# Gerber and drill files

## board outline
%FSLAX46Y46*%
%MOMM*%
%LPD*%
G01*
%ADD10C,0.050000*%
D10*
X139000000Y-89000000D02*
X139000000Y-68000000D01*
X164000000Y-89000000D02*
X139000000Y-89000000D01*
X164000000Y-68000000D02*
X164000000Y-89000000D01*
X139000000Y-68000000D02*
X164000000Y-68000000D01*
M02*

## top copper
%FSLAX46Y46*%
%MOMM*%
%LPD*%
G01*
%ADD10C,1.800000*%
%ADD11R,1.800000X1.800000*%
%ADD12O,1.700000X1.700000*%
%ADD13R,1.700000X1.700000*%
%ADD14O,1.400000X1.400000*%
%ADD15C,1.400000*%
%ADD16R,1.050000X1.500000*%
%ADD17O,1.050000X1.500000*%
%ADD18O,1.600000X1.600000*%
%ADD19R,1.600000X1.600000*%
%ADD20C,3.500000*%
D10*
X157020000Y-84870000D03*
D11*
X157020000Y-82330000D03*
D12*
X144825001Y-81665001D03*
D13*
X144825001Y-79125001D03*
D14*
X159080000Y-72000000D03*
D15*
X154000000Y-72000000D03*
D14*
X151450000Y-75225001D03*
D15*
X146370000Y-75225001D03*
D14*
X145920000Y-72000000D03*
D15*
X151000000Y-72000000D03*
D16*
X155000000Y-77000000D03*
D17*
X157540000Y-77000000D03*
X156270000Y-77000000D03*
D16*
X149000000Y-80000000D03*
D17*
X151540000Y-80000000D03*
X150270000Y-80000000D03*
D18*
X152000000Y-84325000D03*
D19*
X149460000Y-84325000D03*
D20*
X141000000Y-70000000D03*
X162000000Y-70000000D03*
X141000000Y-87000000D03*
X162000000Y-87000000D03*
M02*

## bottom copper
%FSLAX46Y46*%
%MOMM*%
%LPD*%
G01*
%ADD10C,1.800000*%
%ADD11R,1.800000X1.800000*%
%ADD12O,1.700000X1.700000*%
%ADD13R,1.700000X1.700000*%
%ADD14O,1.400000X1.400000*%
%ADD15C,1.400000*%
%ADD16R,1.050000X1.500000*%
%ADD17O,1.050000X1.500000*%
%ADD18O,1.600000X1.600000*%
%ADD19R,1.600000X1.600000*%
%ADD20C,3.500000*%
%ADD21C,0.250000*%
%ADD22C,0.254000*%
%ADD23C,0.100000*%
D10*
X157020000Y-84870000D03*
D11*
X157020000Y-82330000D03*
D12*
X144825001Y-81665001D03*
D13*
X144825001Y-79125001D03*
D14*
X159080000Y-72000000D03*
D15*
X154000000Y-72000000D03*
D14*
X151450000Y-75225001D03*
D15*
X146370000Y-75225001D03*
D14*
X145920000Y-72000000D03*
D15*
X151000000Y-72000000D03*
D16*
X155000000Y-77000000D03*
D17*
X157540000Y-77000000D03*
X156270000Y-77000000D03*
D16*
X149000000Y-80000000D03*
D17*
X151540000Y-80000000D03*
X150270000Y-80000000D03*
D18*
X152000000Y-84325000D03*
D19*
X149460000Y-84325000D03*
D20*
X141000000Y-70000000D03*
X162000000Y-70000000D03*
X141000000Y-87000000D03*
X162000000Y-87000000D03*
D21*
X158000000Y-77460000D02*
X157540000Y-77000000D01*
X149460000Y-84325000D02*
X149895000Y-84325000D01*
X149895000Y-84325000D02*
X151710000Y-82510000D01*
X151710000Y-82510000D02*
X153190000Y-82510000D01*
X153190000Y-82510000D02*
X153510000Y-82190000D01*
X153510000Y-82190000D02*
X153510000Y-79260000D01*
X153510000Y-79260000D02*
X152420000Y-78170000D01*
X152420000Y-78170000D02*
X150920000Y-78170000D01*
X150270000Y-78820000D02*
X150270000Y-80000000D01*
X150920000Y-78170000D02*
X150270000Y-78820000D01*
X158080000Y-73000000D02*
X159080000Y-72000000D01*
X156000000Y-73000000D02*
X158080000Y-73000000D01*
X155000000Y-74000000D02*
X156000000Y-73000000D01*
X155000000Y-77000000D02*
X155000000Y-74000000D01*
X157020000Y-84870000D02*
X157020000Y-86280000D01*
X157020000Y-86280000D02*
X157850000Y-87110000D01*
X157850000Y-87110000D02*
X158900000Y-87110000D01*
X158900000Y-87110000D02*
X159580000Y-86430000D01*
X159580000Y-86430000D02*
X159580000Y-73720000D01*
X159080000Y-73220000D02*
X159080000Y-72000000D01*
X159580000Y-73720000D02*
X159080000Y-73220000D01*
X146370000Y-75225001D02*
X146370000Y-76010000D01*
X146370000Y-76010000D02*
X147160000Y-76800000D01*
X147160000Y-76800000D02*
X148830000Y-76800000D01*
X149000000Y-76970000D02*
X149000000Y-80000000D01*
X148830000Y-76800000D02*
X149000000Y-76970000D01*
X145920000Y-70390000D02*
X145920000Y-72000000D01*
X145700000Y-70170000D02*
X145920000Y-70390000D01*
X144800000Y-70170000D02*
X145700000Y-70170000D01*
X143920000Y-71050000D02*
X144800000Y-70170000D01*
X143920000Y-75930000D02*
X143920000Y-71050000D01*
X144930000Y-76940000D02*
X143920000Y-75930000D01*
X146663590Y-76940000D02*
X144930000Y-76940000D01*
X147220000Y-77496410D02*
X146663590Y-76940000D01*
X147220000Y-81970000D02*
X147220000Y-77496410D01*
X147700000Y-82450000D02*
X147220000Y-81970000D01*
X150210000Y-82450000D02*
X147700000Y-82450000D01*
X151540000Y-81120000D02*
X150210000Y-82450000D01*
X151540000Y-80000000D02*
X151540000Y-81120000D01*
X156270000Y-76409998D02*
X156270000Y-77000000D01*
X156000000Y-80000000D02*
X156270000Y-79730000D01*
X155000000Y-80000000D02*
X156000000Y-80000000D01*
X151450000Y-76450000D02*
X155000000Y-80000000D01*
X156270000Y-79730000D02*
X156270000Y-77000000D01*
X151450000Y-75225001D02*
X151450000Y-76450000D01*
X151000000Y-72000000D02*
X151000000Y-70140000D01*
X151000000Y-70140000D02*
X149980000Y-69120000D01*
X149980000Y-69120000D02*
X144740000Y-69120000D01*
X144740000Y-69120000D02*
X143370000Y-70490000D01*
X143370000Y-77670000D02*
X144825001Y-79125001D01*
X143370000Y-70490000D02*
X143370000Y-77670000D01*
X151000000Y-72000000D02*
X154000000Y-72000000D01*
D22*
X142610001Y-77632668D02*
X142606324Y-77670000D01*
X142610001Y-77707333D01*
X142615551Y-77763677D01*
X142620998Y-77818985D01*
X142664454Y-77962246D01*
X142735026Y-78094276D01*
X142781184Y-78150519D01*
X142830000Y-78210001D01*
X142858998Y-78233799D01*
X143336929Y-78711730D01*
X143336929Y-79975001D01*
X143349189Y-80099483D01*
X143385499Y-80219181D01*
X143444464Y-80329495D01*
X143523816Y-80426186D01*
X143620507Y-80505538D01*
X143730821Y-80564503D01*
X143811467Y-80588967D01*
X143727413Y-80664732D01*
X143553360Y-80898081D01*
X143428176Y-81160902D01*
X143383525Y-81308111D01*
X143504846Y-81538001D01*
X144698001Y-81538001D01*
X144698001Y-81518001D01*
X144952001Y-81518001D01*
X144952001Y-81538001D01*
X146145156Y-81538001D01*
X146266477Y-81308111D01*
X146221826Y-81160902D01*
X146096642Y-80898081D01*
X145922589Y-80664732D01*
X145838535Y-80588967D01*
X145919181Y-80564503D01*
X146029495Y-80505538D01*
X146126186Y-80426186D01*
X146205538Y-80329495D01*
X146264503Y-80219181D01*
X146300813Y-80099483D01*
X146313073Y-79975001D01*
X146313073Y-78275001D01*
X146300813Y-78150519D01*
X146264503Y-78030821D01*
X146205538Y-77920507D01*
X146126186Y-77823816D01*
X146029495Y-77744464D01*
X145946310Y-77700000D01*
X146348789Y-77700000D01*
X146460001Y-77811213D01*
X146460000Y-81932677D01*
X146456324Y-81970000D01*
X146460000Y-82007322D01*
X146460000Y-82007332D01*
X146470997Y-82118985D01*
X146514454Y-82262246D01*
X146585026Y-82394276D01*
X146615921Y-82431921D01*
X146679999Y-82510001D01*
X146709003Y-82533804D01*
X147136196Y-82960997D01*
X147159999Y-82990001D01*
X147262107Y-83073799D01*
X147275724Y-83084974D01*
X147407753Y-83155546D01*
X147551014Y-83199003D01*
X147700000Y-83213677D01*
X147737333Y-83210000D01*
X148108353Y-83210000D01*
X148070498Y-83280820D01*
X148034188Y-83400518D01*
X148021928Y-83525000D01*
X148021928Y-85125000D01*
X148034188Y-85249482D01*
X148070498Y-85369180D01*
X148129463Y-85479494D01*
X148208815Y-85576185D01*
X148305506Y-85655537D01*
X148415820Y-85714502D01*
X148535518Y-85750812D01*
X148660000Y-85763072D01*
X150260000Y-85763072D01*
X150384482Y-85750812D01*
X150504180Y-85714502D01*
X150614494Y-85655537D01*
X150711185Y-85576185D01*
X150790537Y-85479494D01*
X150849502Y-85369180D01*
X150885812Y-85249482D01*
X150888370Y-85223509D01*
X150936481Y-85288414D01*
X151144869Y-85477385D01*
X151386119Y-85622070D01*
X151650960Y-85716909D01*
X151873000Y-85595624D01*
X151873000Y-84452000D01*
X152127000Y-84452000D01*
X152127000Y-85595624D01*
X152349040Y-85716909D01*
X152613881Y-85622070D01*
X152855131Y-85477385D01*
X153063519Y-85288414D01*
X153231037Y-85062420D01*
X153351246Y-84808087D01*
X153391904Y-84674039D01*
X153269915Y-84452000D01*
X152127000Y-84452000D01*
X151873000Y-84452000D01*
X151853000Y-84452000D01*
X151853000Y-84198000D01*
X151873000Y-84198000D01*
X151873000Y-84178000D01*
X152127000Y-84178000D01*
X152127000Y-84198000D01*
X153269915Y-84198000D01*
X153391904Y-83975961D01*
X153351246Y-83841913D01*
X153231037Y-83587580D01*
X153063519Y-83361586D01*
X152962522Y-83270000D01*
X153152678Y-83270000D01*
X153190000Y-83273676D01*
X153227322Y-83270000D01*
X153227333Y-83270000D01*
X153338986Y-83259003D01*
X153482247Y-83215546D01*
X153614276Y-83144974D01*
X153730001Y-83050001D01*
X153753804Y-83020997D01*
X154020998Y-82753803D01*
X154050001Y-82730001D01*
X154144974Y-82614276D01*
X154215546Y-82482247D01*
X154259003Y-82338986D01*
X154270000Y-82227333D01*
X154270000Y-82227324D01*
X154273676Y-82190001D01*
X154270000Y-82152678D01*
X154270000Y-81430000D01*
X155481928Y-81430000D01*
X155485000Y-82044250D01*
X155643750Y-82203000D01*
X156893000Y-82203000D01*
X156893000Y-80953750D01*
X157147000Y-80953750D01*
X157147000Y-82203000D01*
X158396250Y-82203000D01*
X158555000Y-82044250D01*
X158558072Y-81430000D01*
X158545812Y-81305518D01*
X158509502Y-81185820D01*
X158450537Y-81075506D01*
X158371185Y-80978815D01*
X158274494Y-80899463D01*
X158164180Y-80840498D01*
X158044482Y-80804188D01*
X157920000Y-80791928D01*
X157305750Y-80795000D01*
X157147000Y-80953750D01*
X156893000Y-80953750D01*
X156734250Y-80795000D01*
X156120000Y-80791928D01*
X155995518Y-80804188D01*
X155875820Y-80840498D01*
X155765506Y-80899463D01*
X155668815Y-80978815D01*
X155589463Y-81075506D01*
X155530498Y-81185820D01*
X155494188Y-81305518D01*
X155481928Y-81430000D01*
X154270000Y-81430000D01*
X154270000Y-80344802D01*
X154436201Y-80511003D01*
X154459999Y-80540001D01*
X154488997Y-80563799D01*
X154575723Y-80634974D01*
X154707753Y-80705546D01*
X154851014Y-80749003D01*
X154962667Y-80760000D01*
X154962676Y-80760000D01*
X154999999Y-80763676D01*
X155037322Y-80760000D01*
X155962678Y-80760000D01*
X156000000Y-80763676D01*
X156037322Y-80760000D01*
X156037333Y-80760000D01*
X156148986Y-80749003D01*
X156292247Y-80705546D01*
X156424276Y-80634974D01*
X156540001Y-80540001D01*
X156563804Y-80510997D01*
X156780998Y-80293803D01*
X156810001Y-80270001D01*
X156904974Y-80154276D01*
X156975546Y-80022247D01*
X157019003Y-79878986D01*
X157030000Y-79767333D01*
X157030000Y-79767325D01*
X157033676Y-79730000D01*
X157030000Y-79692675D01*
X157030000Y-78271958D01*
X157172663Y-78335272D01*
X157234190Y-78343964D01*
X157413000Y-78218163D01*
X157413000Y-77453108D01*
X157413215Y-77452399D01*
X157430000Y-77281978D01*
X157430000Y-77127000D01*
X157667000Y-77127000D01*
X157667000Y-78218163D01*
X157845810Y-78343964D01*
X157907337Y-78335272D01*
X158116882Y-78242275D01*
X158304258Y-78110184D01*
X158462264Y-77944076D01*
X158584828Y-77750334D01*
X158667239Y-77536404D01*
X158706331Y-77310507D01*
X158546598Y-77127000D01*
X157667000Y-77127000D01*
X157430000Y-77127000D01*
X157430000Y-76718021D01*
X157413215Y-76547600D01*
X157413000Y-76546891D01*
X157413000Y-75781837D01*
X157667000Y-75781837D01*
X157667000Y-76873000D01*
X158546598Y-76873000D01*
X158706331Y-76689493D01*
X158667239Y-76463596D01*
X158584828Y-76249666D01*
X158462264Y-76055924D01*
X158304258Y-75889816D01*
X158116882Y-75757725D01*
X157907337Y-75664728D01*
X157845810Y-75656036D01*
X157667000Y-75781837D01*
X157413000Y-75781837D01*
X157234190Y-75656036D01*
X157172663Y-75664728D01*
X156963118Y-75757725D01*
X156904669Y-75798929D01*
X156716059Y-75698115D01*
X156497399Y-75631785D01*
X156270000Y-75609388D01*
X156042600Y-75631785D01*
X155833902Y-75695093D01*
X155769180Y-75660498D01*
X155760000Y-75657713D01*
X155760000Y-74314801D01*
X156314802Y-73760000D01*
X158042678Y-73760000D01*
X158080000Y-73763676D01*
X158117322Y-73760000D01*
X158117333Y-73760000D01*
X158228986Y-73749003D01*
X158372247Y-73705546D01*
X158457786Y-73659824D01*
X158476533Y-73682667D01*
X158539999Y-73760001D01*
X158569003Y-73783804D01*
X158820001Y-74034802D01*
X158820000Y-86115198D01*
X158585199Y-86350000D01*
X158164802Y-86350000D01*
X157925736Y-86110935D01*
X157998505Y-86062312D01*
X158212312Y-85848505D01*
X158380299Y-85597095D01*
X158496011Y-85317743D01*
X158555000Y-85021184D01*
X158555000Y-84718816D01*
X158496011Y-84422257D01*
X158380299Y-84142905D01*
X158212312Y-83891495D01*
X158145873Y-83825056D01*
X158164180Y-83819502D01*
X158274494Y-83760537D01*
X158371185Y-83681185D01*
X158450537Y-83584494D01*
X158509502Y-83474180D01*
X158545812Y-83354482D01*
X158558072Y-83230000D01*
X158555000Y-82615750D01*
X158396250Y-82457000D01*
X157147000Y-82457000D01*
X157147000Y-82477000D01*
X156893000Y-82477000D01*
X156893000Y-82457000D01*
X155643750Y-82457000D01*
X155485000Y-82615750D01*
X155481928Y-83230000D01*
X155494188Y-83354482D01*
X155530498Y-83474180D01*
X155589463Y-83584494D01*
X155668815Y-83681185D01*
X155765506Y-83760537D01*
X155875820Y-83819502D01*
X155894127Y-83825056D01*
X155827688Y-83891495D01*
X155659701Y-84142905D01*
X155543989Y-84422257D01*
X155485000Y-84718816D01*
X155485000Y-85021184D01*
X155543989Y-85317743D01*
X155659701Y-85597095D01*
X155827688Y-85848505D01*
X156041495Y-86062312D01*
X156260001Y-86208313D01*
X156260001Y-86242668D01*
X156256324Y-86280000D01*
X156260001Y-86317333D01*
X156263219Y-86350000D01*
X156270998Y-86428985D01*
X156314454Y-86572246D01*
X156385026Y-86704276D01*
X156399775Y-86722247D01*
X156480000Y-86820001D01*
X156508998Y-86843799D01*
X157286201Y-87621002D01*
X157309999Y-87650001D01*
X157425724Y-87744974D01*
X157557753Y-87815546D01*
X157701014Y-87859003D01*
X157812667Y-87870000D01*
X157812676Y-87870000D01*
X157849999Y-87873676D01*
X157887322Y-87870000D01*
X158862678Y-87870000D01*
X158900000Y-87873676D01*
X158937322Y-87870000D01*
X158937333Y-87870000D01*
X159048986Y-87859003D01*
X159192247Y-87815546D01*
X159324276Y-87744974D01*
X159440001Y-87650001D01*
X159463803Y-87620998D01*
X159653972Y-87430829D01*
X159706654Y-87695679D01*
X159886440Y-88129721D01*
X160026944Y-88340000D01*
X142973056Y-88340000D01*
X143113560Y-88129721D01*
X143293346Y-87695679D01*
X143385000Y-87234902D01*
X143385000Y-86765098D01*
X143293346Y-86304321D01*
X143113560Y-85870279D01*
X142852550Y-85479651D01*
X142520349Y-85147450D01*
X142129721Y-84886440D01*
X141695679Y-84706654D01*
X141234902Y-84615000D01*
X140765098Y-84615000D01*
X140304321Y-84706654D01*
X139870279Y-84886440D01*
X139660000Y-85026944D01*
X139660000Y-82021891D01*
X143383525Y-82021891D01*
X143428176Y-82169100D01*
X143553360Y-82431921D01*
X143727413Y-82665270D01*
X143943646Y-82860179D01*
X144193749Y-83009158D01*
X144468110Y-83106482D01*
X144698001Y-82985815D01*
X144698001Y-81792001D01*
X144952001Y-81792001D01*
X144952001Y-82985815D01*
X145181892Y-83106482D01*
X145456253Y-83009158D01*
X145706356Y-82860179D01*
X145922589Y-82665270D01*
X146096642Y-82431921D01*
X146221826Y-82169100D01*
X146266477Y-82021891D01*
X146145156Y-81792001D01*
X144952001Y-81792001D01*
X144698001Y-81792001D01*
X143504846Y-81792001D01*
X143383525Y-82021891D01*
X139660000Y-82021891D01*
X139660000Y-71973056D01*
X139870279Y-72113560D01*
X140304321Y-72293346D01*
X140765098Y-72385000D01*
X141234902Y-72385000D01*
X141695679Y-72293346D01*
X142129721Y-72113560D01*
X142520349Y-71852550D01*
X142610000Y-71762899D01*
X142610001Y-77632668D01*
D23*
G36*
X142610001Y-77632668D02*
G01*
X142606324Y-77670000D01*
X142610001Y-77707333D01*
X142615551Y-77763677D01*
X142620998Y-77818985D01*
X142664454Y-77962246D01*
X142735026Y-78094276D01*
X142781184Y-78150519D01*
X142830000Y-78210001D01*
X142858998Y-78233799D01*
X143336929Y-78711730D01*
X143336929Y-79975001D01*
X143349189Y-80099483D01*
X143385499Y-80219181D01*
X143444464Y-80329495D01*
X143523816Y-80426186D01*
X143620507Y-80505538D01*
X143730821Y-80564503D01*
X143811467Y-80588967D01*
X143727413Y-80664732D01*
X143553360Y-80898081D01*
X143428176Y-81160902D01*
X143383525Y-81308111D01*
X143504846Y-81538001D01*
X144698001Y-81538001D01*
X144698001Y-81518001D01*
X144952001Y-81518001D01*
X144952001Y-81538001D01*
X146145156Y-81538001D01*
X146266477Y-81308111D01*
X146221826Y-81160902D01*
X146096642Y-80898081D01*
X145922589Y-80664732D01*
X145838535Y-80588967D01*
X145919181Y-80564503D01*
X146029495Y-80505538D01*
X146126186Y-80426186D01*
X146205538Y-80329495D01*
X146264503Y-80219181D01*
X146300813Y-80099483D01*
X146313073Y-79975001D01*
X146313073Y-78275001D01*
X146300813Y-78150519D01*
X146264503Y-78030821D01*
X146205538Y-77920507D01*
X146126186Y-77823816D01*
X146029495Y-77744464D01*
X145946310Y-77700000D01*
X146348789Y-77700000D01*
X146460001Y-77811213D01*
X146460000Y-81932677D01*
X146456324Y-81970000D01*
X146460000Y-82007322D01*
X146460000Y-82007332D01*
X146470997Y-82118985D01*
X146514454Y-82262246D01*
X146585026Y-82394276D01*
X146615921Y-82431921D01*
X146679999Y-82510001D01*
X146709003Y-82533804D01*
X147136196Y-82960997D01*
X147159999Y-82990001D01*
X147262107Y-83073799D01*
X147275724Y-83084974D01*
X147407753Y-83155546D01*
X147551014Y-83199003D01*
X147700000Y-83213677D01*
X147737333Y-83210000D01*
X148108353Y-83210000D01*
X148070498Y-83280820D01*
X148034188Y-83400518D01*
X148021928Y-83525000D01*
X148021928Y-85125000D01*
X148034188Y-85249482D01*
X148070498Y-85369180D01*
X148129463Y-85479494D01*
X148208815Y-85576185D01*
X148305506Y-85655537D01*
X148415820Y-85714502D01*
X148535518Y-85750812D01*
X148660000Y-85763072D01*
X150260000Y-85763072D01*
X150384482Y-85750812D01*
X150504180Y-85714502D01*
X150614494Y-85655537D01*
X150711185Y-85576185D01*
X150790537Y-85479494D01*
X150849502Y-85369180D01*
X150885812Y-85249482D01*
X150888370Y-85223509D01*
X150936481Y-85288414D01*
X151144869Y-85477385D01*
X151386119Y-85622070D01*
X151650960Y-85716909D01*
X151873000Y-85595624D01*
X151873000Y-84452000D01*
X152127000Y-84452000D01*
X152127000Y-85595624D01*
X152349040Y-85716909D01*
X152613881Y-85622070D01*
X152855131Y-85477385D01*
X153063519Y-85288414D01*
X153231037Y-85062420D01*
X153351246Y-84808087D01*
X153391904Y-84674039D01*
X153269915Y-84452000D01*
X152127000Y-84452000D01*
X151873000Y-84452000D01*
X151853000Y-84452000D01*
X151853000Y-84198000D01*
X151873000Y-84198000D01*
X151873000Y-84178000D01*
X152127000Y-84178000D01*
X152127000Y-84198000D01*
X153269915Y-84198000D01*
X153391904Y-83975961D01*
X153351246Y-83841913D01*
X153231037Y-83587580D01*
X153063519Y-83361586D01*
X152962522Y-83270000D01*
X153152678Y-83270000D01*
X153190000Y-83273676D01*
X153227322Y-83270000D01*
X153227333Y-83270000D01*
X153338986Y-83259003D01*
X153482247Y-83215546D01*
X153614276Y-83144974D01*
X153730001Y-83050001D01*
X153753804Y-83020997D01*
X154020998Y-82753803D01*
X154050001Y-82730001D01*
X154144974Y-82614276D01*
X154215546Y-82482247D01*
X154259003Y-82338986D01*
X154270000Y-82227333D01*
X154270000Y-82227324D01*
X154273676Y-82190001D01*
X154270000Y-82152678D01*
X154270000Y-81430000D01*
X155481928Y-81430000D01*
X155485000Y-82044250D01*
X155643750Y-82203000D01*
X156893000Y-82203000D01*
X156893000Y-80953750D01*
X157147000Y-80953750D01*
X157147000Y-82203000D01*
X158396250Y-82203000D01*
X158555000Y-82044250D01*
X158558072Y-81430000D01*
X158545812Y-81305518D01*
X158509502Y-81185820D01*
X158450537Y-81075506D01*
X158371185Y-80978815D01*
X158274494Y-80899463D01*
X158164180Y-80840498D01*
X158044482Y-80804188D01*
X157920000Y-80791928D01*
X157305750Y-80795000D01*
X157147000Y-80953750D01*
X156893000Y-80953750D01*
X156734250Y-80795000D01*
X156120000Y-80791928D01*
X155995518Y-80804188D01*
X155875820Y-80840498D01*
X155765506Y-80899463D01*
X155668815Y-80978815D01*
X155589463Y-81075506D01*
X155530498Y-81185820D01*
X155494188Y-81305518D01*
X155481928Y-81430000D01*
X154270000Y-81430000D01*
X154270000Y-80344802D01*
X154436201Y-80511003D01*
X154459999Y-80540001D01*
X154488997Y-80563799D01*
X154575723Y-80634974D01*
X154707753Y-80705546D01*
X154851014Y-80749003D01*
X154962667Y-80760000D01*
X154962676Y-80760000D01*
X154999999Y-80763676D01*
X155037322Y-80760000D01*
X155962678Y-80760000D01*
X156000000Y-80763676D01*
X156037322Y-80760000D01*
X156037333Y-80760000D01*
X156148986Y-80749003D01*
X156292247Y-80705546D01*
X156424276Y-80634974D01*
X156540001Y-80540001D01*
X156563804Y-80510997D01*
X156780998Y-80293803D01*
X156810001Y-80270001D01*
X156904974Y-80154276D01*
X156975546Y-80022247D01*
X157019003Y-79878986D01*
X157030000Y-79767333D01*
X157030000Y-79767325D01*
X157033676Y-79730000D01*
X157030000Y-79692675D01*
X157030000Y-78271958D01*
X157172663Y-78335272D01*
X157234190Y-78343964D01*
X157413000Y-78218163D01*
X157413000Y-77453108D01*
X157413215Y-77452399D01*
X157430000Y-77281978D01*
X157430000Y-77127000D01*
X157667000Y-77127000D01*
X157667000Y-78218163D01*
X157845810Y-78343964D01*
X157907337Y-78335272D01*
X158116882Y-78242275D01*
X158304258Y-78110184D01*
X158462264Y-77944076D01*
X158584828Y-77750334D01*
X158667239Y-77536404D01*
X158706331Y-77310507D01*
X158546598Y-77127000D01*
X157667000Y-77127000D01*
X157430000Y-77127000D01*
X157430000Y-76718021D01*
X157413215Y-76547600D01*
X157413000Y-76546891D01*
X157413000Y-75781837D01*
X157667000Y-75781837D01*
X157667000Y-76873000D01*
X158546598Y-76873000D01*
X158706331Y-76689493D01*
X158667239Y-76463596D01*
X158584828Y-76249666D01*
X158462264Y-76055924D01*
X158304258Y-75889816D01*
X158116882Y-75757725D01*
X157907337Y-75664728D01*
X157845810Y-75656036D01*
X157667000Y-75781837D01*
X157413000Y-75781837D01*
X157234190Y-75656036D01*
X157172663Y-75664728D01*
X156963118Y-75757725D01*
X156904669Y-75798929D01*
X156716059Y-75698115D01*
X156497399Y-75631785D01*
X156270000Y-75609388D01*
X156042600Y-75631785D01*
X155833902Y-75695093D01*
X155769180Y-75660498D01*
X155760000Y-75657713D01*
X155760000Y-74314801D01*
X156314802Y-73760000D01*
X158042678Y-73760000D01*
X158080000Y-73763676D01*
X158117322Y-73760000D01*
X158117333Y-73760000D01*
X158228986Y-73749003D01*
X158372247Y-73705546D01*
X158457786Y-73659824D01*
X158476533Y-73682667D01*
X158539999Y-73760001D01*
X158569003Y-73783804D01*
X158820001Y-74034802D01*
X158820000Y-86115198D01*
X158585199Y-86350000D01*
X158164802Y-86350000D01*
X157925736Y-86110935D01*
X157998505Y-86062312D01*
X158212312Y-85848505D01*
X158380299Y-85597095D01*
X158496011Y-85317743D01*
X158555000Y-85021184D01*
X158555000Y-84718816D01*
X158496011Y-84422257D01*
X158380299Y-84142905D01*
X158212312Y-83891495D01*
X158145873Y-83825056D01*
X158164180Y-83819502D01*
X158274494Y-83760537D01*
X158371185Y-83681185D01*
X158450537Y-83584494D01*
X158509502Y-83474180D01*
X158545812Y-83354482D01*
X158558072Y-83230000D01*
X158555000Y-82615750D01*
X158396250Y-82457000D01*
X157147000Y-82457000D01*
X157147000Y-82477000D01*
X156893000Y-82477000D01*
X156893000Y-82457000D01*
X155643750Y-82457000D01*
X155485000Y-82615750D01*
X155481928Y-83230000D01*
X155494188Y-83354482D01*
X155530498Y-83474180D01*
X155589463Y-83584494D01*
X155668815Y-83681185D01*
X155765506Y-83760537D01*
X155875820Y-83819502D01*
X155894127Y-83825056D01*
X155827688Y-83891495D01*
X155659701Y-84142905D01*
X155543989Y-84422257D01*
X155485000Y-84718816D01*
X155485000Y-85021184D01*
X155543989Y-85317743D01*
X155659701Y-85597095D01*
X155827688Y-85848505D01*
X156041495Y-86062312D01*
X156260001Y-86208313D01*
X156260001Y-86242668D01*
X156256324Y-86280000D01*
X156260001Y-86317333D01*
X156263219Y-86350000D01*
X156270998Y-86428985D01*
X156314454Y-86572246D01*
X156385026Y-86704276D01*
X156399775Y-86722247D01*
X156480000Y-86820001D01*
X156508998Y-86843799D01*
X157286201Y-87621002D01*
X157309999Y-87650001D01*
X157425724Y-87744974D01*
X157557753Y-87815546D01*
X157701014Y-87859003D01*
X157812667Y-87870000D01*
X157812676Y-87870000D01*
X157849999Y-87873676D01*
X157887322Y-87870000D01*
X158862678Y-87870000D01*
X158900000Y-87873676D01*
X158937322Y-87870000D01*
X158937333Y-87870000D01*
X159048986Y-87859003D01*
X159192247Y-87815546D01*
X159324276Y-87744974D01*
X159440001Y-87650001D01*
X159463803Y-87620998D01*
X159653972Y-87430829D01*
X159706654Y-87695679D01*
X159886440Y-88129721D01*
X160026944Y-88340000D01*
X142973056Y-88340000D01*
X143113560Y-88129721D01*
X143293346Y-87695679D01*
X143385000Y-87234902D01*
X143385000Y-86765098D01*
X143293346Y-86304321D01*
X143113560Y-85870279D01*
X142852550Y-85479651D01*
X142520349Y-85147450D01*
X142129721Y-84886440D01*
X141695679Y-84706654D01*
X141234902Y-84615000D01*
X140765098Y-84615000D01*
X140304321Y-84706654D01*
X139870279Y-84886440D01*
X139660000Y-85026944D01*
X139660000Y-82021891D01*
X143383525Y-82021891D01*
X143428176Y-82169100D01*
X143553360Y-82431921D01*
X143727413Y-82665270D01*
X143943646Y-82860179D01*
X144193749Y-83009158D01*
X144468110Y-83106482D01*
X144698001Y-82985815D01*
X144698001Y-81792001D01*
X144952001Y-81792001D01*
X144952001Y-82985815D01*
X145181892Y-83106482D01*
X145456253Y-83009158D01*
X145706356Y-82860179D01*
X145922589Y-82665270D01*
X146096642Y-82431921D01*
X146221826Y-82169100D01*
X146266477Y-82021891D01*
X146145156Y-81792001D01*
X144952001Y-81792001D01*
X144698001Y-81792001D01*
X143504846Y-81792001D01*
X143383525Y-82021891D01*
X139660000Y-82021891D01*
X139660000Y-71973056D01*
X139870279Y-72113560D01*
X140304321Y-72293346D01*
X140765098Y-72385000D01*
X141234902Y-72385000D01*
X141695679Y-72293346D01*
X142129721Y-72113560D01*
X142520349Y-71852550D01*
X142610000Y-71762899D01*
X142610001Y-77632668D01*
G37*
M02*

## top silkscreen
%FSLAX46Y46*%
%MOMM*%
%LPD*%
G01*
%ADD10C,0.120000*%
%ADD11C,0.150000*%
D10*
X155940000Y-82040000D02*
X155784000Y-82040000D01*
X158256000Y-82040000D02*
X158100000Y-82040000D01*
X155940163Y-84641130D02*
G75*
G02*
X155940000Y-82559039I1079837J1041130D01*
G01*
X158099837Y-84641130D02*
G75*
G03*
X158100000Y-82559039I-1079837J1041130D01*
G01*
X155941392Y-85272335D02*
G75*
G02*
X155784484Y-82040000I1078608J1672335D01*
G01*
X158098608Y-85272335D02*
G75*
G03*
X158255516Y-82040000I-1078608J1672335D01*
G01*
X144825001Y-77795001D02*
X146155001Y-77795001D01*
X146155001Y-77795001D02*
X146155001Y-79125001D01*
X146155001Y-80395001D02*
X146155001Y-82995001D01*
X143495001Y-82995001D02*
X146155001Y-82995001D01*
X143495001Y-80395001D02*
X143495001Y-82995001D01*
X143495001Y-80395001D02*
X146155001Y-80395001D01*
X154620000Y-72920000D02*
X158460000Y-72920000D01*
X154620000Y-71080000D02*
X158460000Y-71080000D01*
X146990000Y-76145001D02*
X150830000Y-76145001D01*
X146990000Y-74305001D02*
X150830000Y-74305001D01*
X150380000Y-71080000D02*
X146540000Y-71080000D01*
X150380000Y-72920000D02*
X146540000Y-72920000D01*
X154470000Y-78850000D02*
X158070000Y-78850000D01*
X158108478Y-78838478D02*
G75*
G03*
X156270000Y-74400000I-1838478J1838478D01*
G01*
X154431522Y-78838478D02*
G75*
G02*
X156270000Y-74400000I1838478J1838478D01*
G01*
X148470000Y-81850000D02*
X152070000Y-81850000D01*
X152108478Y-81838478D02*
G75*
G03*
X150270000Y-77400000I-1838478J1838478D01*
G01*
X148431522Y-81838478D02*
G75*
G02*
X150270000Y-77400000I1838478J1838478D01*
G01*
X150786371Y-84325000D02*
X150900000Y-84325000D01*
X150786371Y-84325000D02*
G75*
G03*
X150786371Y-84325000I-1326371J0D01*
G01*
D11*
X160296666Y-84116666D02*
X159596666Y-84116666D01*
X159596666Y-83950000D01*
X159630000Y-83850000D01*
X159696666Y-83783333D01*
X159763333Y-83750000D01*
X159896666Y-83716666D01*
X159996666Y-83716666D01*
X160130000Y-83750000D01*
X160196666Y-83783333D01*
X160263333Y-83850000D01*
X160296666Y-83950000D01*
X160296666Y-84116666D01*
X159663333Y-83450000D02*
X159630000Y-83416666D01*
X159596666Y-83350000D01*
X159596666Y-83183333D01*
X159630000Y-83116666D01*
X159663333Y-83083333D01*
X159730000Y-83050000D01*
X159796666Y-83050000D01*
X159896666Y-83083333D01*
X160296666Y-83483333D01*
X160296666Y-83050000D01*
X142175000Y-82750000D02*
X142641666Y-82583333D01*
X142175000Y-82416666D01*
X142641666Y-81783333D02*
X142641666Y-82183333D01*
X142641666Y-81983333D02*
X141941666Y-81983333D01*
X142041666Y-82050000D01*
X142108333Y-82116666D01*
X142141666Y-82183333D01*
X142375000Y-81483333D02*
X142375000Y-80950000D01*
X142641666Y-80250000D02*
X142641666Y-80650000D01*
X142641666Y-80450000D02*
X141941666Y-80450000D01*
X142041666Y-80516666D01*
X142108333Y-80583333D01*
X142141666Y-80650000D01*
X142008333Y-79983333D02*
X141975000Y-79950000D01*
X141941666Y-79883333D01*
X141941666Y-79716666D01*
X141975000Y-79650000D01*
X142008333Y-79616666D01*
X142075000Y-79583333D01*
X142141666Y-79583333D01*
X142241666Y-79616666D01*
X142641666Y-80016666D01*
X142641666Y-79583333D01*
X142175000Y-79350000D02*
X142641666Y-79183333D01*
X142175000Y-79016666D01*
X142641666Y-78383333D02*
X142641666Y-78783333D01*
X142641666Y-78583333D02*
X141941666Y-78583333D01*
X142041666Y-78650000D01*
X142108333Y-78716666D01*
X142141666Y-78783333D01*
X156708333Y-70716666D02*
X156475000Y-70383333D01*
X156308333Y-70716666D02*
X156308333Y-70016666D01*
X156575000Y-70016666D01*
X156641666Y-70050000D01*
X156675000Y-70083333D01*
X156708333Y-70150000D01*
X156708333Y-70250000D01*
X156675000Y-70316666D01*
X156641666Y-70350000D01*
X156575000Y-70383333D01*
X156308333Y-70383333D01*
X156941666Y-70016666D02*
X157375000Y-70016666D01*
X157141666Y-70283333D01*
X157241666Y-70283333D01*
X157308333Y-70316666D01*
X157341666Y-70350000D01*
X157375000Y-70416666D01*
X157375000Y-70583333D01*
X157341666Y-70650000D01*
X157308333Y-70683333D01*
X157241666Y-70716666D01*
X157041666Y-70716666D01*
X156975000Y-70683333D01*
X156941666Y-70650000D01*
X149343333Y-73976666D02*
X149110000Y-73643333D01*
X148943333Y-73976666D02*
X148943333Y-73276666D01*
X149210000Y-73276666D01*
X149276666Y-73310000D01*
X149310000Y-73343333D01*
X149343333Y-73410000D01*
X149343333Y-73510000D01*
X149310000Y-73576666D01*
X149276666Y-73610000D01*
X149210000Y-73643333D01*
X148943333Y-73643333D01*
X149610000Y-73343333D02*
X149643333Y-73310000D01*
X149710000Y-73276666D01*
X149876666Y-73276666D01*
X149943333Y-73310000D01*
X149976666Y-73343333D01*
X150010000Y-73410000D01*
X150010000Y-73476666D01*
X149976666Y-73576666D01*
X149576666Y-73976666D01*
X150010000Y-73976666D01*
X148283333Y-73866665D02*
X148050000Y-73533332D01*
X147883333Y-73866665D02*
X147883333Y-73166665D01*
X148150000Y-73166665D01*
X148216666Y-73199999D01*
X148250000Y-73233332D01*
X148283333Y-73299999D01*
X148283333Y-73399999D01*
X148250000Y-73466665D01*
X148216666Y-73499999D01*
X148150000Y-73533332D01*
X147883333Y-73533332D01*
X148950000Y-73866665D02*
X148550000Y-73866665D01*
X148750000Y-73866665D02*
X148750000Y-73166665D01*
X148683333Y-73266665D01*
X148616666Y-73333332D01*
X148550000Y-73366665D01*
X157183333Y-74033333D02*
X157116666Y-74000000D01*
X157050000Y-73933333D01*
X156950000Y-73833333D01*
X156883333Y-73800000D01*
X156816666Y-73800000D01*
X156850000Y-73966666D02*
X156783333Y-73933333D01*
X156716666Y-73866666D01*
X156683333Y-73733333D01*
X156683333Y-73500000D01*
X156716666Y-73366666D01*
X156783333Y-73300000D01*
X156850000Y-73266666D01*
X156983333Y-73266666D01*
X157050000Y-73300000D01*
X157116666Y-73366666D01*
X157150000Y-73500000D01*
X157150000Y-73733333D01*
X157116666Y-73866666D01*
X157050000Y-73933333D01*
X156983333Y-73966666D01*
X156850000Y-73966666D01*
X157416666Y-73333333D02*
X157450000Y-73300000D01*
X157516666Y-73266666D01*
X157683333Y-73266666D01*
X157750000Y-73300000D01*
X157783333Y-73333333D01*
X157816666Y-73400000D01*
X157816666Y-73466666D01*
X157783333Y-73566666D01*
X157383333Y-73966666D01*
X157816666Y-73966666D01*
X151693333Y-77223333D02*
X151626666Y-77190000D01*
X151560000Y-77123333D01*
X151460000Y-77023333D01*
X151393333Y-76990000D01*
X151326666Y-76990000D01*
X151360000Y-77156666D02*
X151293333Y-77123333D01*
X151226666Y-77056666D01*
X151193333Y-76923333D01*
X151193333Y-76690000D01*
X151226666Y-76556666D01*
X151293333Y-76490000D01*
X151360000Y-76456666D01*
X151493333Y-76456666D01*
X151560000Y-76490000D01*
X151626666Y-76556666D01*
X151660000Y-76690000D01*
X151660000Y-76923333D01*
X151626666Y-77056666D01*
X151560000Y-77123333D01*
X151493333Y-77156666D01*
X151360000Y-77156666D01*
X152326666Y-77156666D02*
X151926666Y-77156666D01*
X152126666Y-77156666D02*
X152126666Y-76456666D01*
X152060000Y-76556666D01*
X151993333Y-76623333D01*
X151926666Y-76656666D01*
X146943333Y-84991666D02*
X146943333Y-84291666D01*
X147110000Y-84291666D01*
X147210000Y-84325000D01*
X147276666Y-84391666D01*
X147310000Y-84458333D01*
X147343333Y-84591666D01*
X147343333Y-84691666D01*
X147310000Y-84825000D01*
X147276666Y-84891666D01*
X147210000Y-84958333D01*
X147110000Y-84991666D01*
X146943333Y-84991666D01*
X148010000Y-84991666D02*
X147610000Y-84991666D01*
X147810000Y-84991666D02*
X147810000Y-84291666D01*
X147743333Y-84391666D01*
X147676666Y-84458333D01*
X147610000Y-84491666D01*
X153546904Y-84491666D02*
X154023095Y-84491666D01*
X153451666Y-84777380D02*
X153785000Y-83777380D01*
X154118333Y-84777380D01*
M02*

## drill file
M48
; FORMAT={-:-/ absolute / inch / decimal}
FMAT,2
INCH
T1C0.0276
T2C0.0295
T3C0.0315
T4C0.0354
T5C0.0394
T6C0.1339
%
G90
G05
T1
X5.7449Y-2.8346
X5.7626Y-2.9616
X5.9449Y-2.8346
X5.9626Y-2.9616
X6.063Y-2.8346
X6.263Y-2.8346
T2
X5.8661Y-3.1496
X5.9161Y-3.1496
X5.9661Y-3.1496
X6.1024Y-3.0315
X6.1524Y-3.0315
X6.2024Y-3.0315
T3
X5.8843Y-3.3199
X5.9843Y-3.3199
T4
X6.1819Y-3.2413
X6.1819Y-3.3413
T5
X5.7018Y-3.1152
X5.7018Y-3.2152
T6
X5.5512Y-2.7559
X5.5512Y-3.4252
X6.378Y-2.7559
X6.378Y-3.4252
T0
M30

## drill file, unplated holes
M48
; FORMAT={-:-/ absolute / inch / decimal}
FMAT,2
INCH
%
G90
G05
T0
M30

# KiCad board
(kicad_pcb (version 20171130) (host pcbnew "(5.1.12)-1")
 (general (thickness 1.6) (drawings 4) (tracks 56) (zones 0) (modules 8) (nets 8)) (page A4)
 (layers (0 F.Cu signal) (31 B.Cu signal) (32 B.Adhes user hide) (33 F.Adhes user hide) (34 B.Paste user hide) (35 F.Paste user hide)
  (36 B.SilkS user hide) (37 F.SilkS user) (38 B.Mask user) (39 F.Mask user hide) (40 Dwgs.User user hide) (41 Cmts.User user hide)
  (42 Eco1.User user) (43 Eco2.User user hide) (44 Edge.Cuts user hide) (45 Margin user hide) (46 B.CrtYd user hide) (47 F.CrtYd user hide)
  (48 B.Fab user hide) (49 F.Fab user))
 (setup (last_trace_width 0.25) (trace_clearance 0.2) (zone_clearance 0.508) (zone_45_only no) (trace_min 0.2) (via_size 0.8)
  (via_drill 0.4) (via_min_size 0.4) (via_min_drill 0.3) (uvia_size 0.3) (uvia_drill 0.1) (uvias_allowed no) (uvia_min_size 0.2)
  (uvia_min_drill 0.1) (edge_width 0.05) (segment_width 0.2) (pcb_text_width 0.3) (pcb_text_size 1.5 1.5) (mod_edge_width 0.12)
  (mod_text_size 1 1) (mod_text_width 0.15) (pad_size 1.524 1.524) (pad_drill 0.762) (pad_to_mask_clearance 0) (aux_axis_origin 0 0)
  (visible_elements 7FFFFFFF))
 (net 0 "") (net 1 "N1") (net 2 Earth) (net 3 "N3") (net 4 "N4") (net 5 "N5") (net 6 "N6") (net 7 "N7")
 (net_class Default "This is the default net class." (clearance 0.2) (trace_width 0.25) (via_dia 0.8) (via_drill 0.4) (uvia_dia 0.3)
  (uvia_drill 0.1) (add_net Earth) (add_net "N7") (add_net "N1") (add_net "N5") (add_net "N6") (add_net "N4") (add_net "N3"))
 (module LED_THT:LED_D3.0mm (layer F.Cu) (at 157.02 82.33 270)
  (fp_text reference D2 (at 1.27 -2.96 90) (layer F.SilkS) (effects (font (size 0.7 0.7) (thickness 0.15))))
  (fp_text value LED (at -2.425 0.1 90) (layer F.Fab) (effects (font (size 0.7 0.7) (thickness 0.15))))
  (fp_line (start -0.29 1.08) (end -0.29 1.236) (layer F.SilkS) (width 0.12))
  (fp_line (start -0.29 -1.236) (end -0.29 -1.08) (layer F.SilkS) (width 0.12))
  (fp_arc (start 1.27 0) (end 0.229039 1.08) (angle -87.9) (layer F.SilkS) (width 0.12))
  (fp_arc (start 1.27 0) (end 0.229039 -1.08) (angle 87.9) (layer F.SilkS) (width 0.12))
  (fp_arc (start 1.27 0) (end -0.29 1.235516) (angle -108.8) (layer F.SilkS) (width 0.12))
  (fp_arc (start 1.27 0) (end -0.29 -1.235516) (angle 108.8) (layer F.SilkS) (width 0.12))
  (pad 2 thru_hole circle (at 2.54 0 270) (size 1.8 1.8) (drill 0.9) (layers *.Cu *.Mask) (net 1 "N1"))
  (pad 1 thru_hole rect (at 0 0 270) (size 1.8 1.8) (drill 0.9) (layers *.Cu *.Mask) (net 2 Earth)))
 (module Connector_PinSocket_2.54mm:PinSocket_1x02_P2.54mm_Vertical (layer F.Cu) (at 144.825001 79.125001)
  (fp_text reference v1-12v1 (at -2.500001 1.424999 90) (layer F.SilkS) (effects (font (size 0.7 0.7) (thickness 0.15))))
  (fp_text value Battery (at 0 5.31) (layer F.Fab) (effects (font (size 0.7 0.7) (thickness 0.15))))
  (fp_line (start 0 -1.33) (end 1.33 -1.33) (layer F.SilkS) (width 0.12))
  (fp_line (start 1.33 -1.33) (end 1.33 0) (layer F.SilkS) (width 0.12))
  (fp_line (start 1.33 1.27) (end 1.33 3.87) (layer F.SilkS) (width 0.12))
  (fp_line (start -1.33 3.87) (end 1.33 3.87) (layer F.SilkS) (width 0.12))
  (fp_line (start -1.33 1.27) (end -1.33 3.87) (layer F.SilkS) (width 0.12))
  (fp_line (start -1.33 1.27) (end 1.33 1.27) (layer F.SilkS) (width 0.12))
  (pad 2 thru_hole oval (at 0 2.54) (size 1.7 1.7) (drill 1) (layers *.Cu *.Mask) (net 2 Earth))
  (pad 1 thru_hole rect (at 0 0) (size 1.7 1.7) (drill 1) (layers *.Cu *.Mask) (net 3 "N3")))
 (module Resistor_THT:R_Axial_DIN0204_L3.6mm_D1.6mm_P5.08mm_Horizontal (layer F.Cu) (at 154 72)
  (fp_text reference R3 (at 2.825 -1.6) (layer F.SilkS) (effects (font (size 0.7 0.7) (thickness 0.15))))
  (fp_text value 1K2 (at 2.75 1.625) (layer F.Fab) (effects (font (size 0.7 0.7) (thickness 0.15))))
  (fp_line (start 0.62 0.92) (end 4.46 0.92) (layer F.SilkS) (width 0.12))
  (fp_line (start 0.62 -0.92) (end 4.46 -0.92) (layer F.SilkS) (width 0.12))
  (pad 2 thru_hole oval (at 5.08 0) (size 1.4 1.4) (drill 0.7) (layers *.Cu *.Mask) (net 1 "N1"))
  (pad 1 thru_hole circle (at 0 0) (size 1.4 1.4) (drill 0.7) (layers *.Cu *.Mask) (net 3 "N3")))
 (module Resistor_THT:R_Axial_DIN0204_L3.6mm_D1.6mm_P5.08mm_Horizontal (layer F.Cu) (at 146.37 75.225001)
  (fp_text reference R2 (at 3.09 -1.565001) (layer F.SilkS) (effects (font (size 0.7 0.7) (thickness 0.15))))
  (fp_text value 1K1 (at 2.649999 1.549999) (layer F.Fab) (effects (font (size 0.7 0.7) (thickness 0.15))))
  (fp_line (start 0.62 0.92) (end 4.46 0.92) (layer F.SilkS) (width 0.12))
  (fp_line (start 0.62 -0.92) (end 4.46 -0.92) (layer F.SilkS) (width 0.12))
  (pad 2 thru_hole oval (at 5.08 0) (size 1.4 1.4) (drill 0.7) (layers *.Cu *.Mask) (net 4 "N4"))
  (pad 1 thru_hole circle (at 0 0) (size 1.4 1.4) (drill 0.7) (layers *.Cu *.Mask) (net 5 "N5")))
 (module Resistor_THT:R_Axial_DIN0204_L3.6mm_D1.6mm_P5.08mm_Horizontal (layer F.Cu) (at 151 72 180)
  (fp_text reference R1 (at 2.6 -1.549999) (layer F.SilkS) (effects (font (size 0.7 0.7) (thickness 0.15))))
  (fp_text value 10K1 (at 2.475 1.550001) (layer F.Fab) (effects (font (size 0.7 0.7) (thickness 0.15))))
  (fp_line (start 0.62 0.92) (end 4.46 0.92) (layer F.SilkS) (width 0.12))
  (fp_line (start 0.62 -0.92) (end 4.46 -0.92) (layer F.SilkS) (width 0.12))
  (pad 2 thru_hole oval (at 5.08 0 180) (size 1.4 1.4) (drill 0.7) (layers *.Cu *.Mask) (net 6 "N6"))
  (pad 1 thru_hole circle (at 0 0 180) (size 1.4 1.4) (drill 0.7) (layers *.Cu *.Mask) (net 3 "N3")))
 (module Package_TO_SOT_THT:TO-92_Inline (layer F.Cu) (at 155 77)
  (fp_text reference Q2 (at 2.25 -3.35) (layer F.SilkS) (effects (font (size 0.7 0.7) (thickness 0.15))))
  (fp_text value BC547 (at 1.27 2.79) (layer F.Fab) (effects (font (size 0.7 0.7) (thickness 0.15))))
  (fp_line (start -0.53 1.85) (end 3.07 1.85) (layer F.SilkS) (width 0.12))
  (fp_arc (start 1.27 0) (end 1.27 -2.6) (angle 135) (layer F.SilkS) (width 0.12))
  (fp_arc (start 1.27 0) (end 1.27 -2.6) (angle -135) (layer F.SilkS) (width 0.12))
  (pad 1 thru_hole rect (at 0 0) (size 1.05 1.5) (drill 0.75) (layers *.Cu *.Mask) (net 1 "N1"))
  (pad 3 thru_hole oval (at 2.54 0) (size 1.05 1.5) (drill 0.75) (layers *.Cu *.Mask) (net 2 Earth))
  (pad 2 thru_hole oval (at 1.27 0) (size 1.05 1.5) (drill 0.75) (layers *.Cu *.Mask) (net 4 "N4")))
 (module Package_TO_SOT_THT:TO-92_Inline (layer F.Cu) (at 149 80)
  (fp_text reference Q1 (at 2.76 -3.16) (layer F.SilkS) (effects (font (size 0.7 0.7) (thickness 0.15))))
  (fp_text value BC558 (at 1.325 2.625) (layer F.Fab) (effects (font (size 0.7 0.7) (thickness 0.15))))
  (fp_line (start -0.53 1.85) (end 3.07 1.85) (layer F.SilkS) (width 0.12))
  (fp_arc (start 1.27 0) (end 1.27 -2.6) (angle 135) (layer F.SilkS) (width 0.12))
  (fp_arc (start 1.27 0) (end 1.27 -2.6) (angle -135) (layer F.SilkS) (width 0.12))
  (pad 1 thru_hole rect (at 0 0) (size 1.05 1.5) (drill 0.75) (layers *.Cu *.Mask) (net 5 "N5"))
  (pad 3 thru_hole oval (at 2.54 0) (size 1.05 1.5) (drill 0.75) (layers *.Cu *.Mask) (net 6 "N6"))
  (pad 2 thru_hole oval (at 1.27 0) (size 1.05 1.5) (drill 0.75) (layers *.Cu *.Mask) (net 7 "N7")))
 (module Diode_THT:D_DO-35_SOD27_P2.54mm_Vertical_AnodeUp (layer F.Cu) (at 149.46 84.325)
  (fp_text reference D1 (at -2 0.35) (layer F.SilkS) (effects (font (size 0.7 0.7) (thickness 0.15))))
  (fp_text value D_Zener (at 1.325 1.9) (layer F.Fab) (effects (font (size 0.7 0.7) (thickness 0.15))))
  (fp_line (start 1.326371 0) (end 1.44 0) (layer F.SilkS) (width 0.12))
  (fp_circle (center 0 0) (end 1.326371 0) (layer F.SilkS) (width 0.12))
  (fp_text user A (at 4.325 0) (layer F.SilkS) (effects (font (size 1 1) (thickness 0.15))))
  (pad 2 thru_hole oval (at 2.54 0) (size 1.6 1.6) (drill 0.8) (layers *.Cu *.Mask) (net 2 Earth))
  (pad 1 thru_hole rect (at 0 0) (size 1.6 1.6) (drill 0.8) (layers *.Cu *.Mask) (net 7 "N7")))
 (gr_line (start 139 89) (end 139 68) (layer Edge.Cuts) (width 0.05))
 (gr_line (start 164 89) (end 139 89) (layer Edge.Cuts) (width 0.05))
 (gr_line (start 164 68) (end 164 89) (layer Edge.Cuts) (width 0.05))
 (gr_line (start 139 68) (end 164 68) (layer Edge.Cuts) (width 0.05))
 (via (at 141 70) (size 3.5) (drill 3.4) (layers F.Cu B.Cu) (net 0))
 (via (at 162 70) (size 3.5) (drill 3.4) (layers F.Cu B.Cu) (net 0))
 (via (at 141 87) (size 3.5) (drill 3.4) (layers F.Cu B.Cu) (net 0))
 (via (at 162 87) (size 3.5) (drill 3.4) (layers F.Cu B.Cu) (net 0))
 (segment (start 158 77.46) (end 157.54 77) (width 0.25) (layer B.Cu) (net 2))
 (segment (start 149.46 84.325) (end 149.895 84.325) (width 0.25) (layer B.Cu) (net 7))
 (segment (start 149.895 84.325) (end 151.71 82.51) (width 0.25) (layer B.Cu) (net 7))
 (segment (start 151.71 82.51) (end 153.19 82.51) (width 0.25) (layer B.Cu) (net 7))
 (segment (start 153.19 82.51) (end 153.51 82.19) (width 0.25) (layer B.Cu) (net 7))
 (segment (start 153.51 82.19) (end 153.51 79.26) (width 0.25) (layer B.Cu) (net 7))
 (segment (start 153.51 79.26) (end 152.42 78.17) (width 0.25) (layer B.Cu) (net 7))
 (segment (start 152.42 78.17) (end 150.92 78.17) (width 0.25) (layer B.Cu) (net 7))
 (segment (start 150.27 78.82) (end 150.27 80) (width 0.25) (layer B.Cu) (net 7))
 (segment (start 150.92 78.17) (end 150.27 78.82) (width 0.25) (layer B.Cu) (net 7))
 (segment (start 158.08 73) (end 159.08 72) (width 0.25) (layer B.Cu) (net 1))
 (segment (start 156 73) (end 158.08 73) (width 0.25) (layer B.Cu) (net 1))
 (segment (start 155 74) (end 156 73) (width 0.25) (layer B.Cu) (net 1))
 (segment (start 155 77) (end 155 74) (width 0.25) (layer B.Cu) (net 1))
 (segment (start 157.02 84.87) (end 157.02 86.28) (width 0.25) (layer B.Cu) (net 1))
 (segment (start 157.02 86.28) (end 157.85 87.11) (width 0.25) (layer B.Cu) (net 1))
 (segment (start 157.85 87.11) (end 158.9 87.11) (width 0.25) (layer B.Cu) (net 1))
 (segment (start 158.9 87.11) (end 159.58 86.43) (width 0.25) (layer B.Cu) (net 1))
 (segment (start 159.58 86.43) (end 159.58 73.72) (width 0.25) (layer B.Cu) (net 1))
 (segment (start 159.08 73.22) (end 159.08 72) (width 0.25) (layer B.Cu) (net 1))
 (segment (start 159.58 73.72) (end 159.08 73.22) (width 0.25) (layer B.Cu) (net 1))
 (segment (start 146.37 75.225001) (end 146.37 76.01) (width 0.25) (layer B.Cu) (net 5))
 (segment (start 146.37 76.01) (end 147.16 76.8) (width 0.25) (layer B.Cu) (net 5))
 (segment (start 147.16 76.8) (end 148.83 76.8) (width 0.25) (layer B.Cu) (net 5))
 (segment (start 149 76.97) (end 149 80) (width 0.25) (layer B.Cu) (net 5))
 (segment (start 148.83 76.8) (end 149 76.97) (width 0.25) (layer B.Cu) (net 5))
 (segment (start 145.92 70.39) (end 145.92 72) (width 0.25) (layer B.Cu) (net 6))
 (segment (start 145.7 70.17) (end 145.92 70.39) (width 0.25) (layer B.Cu) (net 6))
 (segment (start 144.8 70.17) (end 145.7 70.17) (width 0.25) (layer B.Cu) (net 6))
 (segment (start 143.92 71.05) (end 144.8 70.17) (width 0.25) (layer B.Cu) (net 6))
 (segment (start 143.92 75.93) (end 143.92 71.05) (width 0.25) (layer B.Cu) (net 6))
 (segment (start 144.93 76.94) (end 143.92 75.93) (width 0.25) (layer B.Cu) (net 6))
 (segment (start 146.66359 76.94) (end 144.93 76.94) (width 0.25) (layer B.Cu) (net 6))
 (segment (start 147.22 77.49641) (end 146.66359 76.94) (width 0.25) (layer B.Cu) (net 6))
 (segment (start 147.22 81.97) (end 147.22 77.49641) (width 0.25) (layer B.Cu) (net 6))
 (segment (start 147.7 82.45) (end 147.22 81.97) (width 0.25) (layer B.Cu) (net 6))
 (segment (start 150.21 82.45) (end 147.7 82.45) (width 0.25) (layer B.Cu) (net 6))
 (segment (start 151.54 81.12) (end 150.21 82.45) (width 0.25) (layer B.Cu) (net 6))
 (segment (start 151.54 80) (end 151.54 81.12) (width 0.25) (layer B.Cu) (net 6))
 (segment (start 156.27 76.409998) (end 156.27 77) (width 0.25) (layer B.Cu) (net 4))
 (segment (start 156 80) (end 156.27 79.73) (width 0.25) (layer B.Cu) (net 4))
 (segment (start 155 80) (end 156 80) (width 0.25) (layer B.Cu) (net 4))
 (segment (start 151.45 76.45) (end 155 80) (width 0.25) (layer B.Cu) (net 4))
 (segment (start 156.27 79.73) (end 156.27 77) (width 0.25) (layer B.Cu) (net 4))
 (segment (start 151.45 75.225001) (end 151.45 76.45) (width 0.25) (layer B.Cu) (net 4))
 (segment (start 151 72) (end 151 70.14) (width 0.25) (layer B.Cu) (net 3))
 (segment (start 151 70.14) (end 149.98 69.12) (width 0.25) (layer B.Cu) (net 3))
 (segment (start 149.98 69.12) (end 144.74 69.12) (width 0.25) (layer B.Cu) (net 3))
 (segment (start 144.74 69.12) (end 143.37 70.49) (width 0.25) (layer B.Cu) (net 3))
 (segment (start 143.37 77.67) (end 144.825001 79.125001) (width 0.25) (layer B.Cu) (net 3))
 (segment (start 143.37 70.49) (end 143.37 77.67) (width 0.25) (layer B.Cu) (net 3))
 (segment (start 151 72) (end 154 72) (width 0.25) (layer B.Cu) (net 3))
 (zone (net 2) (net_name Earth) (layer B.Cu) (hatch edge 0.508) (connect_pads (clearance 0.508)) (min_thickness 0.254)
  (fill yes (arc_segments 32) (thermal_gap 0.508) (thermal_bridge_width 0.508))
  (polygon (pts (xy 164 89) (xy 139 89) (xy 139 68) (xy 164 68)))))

